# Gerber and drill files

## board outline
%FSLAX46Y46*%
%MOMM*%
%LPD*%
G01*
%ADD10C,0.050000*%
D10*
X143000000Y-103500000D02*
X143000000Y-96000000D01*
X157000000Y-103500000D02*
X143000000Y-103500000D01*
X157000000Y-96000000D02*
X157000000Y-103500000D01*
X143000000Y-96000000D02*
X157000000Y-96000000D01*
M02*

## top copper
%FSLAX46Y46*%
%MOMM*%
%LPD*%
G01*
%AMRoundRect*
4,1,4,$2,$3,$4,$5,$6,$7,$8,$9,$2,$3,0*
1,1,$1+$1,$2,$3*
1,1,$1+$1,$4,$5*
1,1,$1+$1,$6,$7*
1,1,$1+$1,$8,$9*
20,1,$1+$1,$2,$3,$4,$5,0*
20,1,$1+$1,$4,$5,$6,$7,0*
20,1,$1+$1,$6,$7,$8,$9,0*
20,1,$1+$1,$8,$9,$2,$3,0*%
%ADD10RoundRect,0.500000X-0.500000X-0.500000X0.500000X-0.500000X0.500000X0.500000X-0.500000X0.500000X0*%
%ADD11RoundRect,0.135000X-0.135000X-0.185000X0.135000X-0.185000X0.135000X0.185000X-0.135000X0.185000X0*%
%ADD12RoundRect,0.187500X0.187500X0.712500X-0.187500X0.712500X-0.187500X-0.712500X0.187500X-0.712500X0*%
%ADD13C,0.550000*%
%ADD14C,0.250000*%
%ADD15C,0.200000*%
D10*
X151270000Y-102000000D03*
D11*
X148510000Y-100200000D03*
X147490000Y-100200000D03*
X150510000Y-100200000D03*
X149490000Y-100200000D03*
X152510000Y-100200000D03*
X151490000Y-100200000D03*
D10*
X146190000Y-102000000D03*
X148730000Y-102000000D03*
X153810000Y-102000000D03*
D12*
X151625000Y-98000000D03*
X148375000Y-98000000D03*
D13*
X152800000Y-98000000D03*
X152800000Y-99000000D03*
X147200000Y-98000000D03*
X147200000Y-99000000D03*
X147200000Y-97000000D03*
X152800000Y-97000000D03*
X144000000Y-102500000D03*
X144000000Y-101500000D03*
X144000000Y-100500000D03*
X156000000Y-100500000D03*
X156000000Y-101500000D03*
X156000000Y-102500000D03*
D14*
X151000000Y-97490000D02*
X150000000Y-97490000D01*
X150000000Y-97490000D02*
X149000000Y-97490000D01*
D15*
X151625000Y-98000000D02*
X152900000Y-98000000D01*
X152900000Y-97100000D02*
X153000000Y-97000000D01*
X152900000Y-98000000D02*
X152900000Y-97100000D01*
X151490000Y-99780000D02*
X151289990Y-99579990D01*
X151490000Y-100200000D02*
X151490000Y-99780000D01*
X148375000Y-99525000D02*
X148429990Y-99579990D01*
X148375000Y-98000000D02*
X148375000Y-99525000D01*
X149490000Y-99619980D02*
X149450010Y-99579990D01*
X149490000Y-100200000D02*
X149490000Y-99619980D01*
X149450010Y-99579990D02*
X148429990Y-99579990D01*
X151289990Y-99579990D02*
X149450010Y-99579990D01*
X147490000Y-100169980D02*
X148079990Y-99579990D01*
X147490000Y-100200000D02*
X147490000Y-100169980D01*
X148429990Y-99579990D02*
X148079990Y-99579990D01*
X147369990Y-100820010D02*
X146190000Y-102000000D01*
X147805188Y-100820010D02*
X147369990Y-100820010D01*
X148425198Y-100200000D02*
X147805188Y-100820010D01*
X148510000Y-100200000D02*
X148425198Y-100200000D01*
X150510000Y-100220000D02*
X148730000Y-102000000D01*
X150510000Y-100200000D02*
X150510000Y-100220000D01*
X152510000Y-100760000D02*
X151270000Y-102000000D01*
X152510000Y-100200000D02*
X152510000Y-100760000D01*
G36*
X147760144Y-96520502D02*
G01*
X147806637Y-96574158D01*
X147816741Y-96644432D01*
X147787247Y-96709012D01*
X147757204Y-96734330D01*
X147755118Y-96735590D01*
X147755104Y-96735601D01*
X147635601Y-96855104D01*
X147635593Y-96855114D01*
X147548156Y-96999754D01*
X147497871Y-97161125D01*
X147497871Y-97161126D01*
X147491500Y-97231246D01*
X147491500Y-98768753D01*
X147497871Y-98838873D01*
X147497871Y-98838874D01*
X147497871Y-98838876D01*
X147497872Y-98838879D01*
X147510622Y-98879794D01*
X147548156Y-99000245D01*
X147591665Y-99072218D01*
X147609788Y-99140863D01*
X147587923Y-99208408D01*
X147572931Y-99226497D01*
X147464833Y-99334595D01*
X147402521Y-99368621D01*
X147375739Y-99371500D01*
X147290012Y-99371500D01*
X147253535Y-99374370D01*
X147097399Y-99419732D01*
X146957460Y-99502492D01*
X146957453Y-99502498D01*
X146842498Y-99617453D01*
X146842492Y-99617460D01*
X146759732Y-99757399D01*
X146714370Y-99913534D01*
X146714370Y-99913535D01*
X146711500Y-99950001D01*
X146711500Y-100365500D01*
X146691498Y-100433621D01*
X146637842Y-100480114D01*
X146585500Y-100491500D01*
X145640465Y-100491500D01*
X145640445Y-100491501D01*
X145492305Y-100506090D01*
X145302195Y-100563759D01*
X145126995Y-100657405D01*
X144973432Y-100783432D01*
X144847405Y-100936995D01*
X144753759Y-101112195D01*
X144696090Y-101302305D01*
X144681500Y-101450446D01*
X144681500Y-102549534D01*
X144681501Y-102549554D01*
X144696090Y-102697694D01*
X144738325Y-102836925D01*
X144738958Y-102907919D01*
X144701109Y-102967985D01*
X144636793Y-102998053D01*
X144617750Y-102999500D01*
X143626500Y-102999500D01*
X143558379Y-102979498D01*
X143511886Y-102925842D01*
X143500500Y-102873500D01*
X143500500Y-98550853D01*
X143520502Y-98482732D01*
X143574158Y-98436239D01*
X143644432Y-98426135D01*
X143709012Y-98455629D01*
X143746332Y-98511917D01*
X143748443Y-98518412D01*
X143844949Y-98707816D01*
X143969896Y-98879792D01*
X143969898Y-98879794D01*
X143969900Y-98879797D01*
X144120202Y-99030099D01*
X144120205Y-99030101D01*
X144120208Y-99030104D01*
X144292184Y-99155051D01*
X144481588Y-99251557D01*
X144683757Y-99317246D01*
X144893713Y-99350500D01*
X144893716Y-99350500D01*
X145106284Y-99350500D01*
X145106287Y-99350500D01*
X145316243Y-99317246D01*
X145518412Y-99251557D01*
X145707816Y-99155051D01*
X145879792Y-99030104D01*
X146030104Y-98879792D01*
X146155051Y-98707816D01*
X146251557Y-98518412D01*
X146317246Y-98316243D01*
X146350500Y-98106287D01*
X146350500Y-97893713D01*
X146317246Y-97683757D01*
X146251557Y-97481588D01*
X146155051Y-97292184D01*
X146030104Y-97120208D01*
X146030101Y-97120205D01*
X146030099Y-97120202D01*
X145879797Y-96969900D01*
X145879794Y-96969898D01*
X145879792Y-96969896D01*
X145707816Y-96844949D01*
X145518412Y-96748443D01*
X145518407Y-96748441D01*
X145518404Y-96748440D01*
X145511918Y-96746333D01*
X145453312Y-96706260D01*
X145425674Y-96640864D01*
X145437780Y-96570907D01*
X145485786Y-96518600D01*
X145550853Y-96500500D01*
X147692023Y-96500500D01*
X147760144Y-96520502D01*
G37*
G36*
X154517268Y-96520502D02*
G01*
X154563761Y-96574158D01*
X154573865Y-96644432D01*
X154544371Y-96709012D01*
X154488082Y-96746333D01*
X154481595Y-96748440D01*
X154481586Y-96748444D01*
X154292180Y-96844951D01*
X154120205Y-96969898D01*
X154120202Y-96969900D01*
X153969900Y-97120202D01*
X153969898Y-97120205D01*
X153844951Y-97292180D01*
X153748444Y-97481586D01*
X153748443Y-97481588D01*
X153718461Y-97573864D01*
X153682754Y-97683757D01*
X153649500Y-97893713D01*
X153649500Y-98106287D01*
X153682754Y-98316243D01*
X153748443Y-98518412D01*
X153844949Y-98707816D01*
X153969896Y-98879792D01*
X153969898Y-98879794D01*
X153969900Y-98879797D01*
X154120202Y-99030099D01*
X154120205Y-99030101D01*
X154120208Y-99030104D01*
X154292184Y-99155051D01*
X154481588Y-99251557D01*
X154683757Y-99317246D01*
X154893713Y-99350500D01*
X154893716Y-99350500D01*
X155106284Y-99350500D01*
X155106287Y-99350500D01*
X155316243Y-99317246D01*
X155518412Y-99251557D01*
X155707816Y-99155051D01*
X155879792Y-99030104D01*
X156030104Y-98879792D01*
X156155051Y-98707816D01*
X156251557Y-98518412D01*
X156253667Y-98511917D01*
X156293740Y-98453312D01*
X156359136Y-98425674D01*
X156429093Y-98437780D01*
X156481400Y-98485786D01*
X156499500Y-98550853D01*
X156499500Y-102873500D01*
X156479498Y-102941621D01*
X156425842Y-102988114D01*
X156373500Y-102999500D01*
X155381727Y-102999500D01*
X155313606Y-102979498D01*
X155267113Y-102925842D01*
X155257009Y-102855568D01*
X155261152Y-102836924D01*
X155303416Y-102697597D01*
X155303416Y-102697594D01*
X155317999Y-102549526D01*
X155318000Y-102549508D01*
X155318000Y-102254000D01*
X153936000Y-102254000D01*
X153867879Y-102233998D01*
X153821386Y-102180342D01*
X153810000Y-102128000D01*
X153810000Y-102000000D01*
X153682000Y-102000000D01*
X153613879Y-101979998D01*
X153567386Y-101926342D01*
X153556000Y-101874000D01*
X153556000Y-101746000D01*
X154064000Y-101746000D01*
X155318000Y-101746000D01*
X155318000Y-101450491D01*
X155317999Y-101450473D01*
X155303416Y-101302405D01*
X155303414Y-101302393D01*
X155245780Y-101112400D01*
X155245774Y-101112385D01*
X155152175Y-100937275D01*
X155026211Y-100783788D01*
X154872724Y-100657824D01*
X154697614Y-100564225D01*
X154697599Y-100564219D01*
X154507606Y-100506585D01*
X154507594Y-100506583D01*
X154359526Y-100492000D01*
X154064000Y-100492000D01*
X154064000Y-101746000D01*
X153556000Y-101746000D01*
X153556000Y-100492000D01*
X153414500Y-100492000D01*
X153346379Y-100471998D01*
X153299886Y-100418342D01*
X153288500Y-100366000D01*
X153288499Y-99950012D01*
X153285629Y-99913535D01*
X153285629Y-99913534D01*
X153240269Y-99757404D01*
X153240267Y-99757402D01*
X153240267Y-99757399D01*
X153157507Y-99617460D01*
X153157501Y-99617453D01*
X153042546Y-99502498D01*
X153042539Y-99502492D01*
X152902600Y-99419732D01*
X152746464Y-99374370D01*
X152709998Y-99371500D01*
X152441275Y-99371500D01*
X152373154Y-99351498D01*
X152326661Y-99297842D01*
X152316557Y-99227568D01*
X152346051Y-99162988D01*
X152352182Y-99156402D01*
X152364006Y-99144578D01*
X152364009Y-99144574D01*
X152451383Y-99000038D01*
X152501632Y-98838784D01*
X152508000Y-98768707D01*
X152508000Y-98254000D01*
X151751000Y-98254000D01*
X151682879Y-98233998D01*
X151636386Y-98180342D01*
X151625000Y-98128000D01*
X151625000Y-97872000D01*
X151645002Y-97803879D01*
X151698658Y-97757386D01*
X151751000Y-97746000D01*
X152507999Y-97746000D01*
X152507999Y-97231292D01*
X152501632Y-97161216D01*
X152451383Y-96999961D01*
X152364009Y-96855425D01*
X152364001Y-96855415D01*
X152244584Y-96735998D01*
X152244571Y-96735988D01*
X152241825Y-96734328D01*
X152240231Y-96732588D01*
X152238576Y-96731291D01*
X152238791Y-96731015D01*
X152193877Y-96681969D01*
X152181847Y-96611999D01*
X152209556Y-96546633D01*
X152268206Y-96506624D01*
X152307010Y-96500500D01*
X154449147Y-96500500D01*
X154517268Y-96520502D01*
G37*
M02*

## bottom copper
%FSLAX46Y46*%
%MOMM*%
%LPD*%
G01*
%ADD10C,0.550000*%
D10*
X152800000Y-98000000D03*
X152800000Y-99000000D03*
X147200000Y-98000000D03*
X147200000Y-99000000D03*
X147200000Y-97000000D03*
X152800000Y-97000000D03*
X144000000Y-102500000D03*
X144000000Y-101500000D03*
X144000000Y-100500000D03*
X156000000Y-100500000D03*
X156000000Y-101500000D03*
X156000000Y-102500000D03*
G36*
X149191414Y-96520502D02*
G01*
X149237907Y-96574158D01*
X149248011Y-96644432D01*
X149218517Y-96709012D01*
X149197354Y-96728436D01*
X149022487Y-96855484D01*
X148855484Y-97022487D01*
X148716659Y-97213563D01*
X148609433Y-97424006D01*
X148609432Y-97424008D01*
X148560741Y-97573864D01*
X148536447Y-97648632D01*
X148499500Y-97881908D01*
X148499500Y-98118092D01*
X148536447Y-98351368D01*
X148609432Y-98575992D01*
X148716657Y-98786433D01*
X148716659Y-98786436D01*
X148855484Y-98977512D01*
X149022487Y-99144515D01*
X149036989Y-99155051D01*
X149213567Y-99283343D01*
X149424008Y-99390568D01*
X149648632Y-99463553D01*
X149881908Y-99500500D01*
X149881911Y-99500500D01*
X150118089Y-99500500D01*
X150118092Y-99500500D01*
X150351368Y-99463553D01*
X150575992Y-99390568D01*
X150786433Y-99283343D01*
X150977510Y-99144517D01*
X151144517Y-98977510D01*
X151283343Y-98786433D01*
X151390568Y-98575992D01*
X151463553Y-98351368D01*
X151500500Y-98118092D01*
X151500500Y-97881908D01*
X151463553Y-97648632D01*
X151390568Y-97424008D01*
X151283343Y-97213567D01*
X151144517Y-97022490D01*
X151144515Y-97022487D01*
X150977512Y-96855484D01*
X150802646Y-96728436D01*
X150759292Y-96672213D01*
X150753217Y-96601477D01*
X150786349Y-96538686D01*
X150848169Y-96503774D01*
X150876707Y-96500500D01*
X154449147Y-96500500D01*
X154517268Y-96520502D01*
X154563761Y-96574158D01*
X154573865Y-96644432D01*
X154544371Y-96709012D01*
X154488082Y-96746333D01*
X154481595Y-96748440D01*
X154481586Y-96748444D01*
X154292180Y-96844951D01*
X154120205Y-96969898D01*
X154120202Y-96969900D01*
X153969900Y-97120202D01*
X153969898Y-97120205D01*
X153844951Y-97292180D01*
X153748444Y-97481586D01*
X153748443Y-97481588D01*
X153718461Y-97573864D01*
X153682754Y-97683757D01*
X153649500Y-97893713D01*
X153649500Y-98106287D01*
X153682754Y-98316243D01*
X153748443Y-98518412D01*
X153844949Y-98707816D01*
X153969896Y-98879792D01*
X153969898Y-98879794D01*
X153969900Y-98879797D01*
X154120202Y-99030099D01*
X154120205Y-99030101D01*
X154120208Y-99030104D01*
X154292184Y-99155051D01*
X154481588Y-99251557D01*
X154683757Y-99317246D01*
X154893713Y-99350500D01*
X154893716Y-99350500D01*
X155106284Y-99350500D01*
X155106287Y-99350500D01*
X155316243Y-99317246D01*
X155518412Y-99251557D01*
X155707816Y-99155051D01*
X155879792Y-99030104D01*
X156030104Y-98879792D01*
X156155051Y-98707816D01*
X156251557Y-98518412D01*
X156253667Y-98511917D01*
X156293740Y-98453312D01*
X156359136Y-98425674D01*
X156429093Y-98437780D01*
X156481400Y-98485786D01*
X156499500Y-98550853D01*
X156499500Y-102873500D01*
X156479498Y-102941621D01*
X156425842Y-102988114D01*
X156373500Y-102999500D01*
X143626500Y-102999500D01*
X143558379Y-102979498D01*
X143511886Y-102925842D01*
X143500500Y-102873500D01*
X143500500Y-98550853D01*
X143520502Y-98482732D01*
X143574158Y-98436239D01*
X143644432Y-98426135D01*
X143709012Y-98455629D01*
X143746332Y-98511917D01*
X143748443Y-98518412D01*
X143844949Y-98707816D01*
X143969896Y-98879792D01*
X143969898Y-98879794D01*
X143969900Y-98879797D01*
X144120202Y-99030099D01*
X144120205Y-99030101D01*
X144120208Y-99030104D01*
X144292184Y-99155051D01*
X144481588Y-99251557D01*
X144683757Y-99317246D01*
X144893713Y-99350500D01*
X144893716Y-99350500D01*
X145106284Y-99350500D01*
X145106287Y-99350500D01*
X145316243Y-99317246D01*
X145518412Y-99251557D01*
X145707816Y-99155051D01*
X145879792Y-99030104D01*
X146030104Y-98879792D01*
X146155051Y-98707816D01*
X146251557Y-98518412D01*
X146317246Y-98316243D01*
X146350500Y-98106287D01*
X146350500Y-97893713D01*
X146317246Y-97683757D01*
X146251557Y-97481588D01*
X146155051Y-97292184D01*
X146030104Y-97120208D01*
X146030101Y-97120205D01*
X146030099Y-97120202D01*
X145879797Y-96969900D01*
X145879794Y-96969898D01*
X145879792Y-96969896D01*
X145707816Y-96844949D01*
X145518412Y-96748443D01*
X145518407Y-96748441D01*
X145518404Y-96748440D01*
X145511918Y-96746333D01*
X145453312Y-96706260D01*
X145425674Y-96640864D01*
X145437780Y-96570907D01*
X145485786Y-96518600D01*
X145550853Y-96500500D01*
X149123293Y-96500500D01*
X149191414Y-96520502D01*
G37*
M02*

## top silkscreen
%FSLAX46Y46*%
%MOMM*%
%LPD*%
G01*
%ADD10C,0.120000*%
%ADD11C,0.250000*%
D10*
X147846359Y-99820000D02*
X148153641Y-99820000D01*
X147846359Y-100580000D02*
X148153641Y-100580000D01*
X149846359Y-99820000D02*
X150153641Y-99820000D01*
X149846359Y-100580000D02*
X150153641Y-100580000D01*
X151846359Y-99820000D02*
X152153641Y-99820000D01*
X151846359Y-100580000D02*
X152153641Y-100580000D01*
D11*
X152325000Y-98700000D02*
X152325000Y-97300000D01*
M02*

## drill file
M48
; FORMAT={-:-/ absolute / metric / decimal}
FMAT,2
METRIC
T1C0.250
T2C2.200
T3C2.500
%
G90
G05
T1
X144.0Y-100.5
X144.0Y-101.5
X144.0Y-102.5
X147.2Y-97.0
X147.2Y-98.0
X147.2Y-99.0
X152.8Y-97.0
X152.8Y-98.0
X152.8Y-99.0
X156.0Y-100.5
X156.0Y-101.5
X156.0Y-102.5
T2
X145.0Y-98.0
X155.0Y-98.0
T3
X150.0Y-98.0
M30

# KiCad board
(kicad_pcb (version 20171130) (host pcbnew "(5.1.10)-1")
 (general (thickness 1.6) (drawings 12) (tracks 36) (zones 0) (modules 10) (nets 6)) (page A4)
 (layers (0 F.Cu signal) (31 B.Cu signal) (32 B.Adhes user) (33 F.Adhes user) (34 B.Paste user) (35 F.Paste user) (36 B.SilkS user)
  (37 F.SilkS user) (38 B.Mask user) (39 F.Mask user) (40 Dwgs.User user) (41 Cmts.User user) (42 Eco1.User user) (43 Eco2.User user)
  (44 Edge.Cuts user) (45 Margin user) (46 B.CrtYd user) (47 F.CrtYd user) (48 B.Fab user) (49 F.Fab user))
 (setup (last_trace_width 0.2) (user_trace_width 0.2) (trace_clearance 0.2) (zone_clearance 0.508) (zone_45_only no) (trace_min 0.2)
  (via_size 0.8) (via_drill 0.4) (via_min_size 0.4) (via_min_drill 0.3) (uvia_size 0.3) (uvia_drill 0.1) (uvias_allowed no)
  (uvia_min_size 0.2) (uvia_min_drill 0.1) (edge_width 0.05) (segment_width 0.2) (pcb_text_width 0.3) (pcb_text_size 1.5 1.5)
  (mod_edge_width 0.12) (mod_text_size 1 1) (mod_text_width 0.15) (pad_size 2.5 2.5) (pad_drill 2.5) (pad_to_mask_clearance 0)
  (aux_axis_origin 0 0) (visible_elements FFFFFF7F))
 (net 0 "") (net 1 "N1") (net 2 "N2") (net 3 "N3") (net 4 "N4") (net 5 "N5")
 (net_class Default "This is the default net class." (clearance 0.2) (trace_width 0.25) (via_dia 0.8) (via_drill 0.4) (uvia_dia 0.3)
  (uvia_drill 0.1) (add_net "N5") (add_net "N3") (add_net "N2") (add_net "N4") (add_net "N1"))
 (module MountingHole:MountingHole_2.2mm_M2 (layer F.Cu) (at 145 98)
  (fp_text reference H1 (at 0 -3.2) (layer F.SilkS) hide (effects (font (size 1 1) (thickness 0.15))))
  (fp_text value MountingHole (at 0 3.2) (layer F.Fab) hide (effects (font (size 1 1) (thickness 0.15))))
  (pad 1 np_thru_hole circle (at 0 0) (size 2.2 2.2) (drill 2.2) (layers *.Cu *.Mask)))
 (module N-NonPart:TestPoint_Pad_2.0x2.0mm (layer F.Cu) (at 151.27 102)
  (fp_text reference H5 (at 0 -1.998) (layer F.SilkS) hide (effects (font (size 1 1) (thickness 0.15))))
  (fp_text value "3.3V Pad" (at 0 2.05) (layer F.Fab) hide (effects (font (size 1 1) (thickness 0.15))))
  (pad 1 smd roundrect (at 0 0) (size 2 2) (layers F.Cu F.Mask) (roundrect_rratio 0.25) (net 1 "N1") (solder_mask_margin 0.05)))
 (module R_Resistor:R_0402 (layer F.Cu) (at 148 100.2)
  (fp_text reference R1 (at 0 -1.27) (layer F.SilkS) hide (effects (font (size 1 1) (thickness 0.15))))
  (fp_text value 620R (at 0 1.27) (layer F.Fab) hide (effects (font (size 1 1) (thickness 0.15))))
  (fp_line (start -0.153641 -0.38) (end 0.153641 -0.38) (layer F.SilkS) (width 0.12))
  (fp_line (start -0.153641 0.38) (end 0.153641 0.38) (layer F.SilkS) (width 0.12))
  (pad 2 smd roundrect (at 0.51 0) (size 0.54 0.64) (layers F.Cu F.Paste F.Mask) (roundrect_rratio 0.25) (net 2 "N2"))
  (pad 1 smd roundrect (at -0.51 0) (size 0.54 0.64) (layers F.Cu F.Paste F.Mask) (roundrect_rratio 0.25) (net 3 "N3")))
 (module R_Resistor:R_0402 (layer F.Cu) (at 150 100.2)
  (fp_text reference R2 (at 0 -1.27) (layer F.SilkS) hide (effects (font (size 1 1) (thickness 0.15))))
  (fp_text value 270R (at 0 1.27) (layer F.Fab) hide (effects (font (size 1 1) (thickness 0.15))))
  (fp_line (start -0.153641 -0.38) (end 0.153641 -0.38) (layer F.SilkS) (width 0.12))
  (fp_line (start -0.153641 0.38) (end 0.153641 0.38) (layer F.SilkS) (width 0.12))
  (pad 2 smd roundrect (at 0.51 0) (size 0.54 0.64) (layers F.Cu F.Paste F.Mask) (roundrect_rratio 0.25) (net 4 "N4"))
  (pad 1 smd roundrect (at -0.51 0) (size 0.54 0.64) (layers F.Cu F.Paste F.Mask) (roundrect_rratio 0.25) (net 3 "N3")))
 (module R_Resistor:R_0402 (layer F.Cu) (at 152 100.2)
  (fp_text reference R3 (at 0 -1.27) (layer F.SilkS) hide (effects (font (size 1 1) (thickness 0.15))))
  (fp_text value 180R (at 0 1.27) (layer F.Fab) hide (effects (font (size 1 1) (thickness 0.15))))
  (fp_line (start -0.153641 -0.38) (end 0.153641 -0.38) (layer F.SilkS) (width 0.12))
  (fp_line (start -0.153641 0.38) (end 0.153641 0.38) (layer F.SilkS) (width 0.12))
  (pad 2 smd roundrect (at 0.51 0) (size 0.54 0.64) (layers F.Cu F.Paste F.Mask) (roundrect_rratio 0.25) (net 1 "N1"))
  (pad 1 smd roundrect (at -0.51 0) (size 0.54 0.64) (layers F.Cu F.Paste F.Mask) (roundrect_rratio 0.25) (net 3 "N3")))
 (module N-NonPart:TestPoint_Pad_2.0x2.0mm (layer F.Cu) (at 146.19 102)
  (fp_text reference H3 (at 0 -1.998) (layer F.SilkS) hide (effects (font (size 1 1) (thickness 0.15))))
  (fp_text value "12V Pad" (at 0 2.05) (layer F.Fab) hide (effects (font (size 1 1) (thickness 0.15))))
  (pad 1 smd roundrect (at 0 0) (size 2 2) (layers F.Cu F.Mask) (roundrect_rratio 0.25) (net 2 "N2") (solder_mask_margin 0.05)))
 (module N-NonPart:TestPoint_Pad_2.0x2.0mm (layer F.Cu) (at 148.73 102)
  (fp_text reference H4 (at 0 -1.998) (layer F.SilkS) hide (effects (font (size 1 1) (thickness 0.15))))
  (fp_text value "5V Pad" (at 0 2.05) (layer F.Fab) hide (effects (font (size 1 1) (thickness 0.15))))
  (pad 1 smd roundrect (at 0 0) (size 2 2) (layers F.Cu F.Mask) (roundrect_rratio 0.25) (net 4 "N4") (solder_mask_margin 0.05)))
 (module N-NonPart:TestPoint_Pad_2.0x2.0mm (layer F.Cu) (at 153.81 102)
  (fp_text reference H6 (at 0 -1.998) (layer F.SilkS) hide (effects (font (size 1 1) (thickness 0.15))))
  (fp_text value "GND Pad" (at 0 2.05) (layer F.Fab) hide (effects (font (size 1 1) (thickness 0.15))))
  (pad 1 smd roundrect (at 0 0) (size 2 2) (layers F.Cu F.Mask) (roundrect_rratio 0.25) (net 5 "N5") (solder_mask_margin 0.05)))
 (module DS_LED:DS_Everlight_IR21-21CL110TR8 (layer F.Cu) (at 150 98 180)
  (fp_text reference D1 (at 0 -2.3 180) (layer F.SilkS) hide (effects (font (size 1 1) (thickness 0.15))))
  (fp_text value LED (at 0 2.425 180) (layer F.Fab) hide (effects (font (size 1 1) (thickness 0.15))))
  (fp_line (start -2.325 -0.7) (end -2.325 0.7) (layer F.SilkS) (width 0.25))
  (pad "" np_thru_hole circle (at 0 0 180) (size 2.5 2.5) (drill 2.5) (layers *.Cu *.Mask) (solder_mask_margin 0.05))
  (pad 1 smd roundrect (at -1.625 0 180) (size 0.75 1.8) (layers F.Cu F.Paste F.Mask) (roundrect_rratio 0.25) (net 5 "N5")
   (solder_mask_margin 0.05) (solder_paste_margin -0.05))
  (pad 2 smd roundrect (at 1.625 0 180) (size 0.75 1.8) (layers F.Cu F.Paste F.Mask) (roundrect_rratio 0.25) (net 3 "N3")
   (solder_mask_margin 0.05) (solder_paste_margin -0.05)))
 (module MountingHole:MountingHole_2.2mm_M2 (layer F.Cu) (at 155 98)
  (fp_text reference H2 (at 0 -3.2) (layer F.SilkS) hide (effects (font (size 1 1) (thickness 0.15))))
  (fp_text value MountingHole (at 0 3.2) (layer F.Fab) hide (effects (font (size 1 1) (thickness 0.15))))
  (pad 1 np_thru_hole circle (at 0 0) (size 2.2 2.2) (drill 2.2) (layers *.Cu *.Mask)))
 (gr_line (start 143 103.5) (end 143 96) (layer Edge.Cuts) (width 0.05))
 (gr_line (start 157 103.5) (end 143 103.5) (layer Edge.Cuts) (width 0.05))
 (gr_line (start 157 96) (end 157 103.5) (layer Edge.Cuts) (width 0.05))
 (gr_line (start 143 96) (end 157 96) (layer Edge.Cuts) (width 0.05))
 (segment (start 151 97.49) (end 150 97.49) (width 0.25) (layer F.Cu) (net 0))
 (segment (start 150 97.49) (end 149 97.49) (width 0.25) (layer F.Cu) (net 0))
 (via (at 152.8 98) (size 0.55) (drill 0.25) (layers F.Cu B.Cu) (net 5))
 (via (at 152.8 99) (size 0.55) (drill 0.25) (layers F.Cu B.Cu) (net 5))
 (via (at 147.2 98) (size 0.55) (drill 0.25) (layers F.Cu B.Cu) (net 5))
 (via (at 147.2 99) (size 0.55) (drill 0.25) (layers F.Cu B.Cu) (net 5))
 (via (at 147.2 97) (size 0.55) (drill 0.25) (layers F.Cu B.Cu) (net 5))
 (via (at 152.8 97) (size 0.55) (drill 0.25) (layers F.Cu B.Cu) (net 5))
 (via (at 144 102.5) (size 0.55) (drill 0.25) (layers F.Cu B.Cu) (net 5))
 (via (at 144 101.5) (size 0.55) (drill 0.25) (layers F.Cu B.Cu) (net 5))
 (via (at 144 100.5) (size 0.55) (drill 0.25) (layers F.Cu B.Cu) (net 5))
 (via (at 156 100.5) (size 0.55) (drill 0.25) (layers F.Cu B.Cu) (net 5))
 (via (at 156 101.5) (size 0.55) (drill 0.25) (layers F.Cu B.Cu) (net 5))
 (via (at 156 102.5) (size 0.55) (drill 0.25) (layers F.Cu B.Cu) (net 5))
 (segment (start 151.625 98) (end 152.9 98) (width 0.2) (layer F.Cu) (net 5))
 (segment (start 152.9 97.1) (end 153 97) (width 0.2) (layer F.Cu) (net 5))
 (segment (start 152.9 98) (end 152.9 97.1) (width 0.2) (layer F.Cu) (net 5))
 (segment (start 151.49 99.78) (end 151.28999 99.57999) (width 0.2) (layer F.Cu) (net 3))
 (segment (start 151.49 100.2) (end 151.49 99.78) (width 0.2) (layer F.Cu) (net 3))
 (segment (start 148.375 99.525) (end 148.42999 99.57999) (width 0.2) (layer F.Cu) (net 3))
 (segment (start 148.375 98) (end 148.375 99.525) (width 0.2) (layer F.Cu) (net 3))
 (segment (start 149.49 99.61998) (end 149.45001 99.57999) (width 0.2) (layer F.Cu) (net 3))
 (segment (start 149.49 100.2) (end 149.49 99.61998) (width 0.2) (layer F.Cu) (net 3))
 (segment (start 149.45001 99.57999) (end 148.42999 99.57999) (width 0.2) (layer F.Cu) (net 3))
 (segment (start 151.28999 99.57999) (end 149.45001 99.57999) (width 0.2) (layer F.Cu) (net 3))
 (segment (start 147.49 100.16998) (end 148.07999 99.57999) (width 0.2) (layer F.Cu) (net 3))
 (segment (start 147.49 100.2) (end 147.49 100.16998) (width 0.2) (layer F.Cu) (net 3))
 (segment (start 148.42999 99.57999) (end 148.07999 99.57999) (width 0.2) (layer F.Cu) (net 3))
 (segment (start 147.36999 100.82001) (end 146.19 102) (width 0.2) (layer F.Cu) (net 2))
 (segment (start 147.805188 100.82001) (end 147.36999 100.82001) (width 0.2) (layer F.Cu) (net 2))
 (segment (start 148.425198 100.2) (end 147.805188 100.82001) (width 0.2) (layer F.Cu) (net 2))
 (segment (start 148.51 100.2) (end 148.425198 100.2) (width 0.2) (layer F.Cu) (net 2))
 (segment (start 150.51 100.22) (end 148.73 102) (width 0.2) (layer F.Cu) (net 4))
 (segment (start 150.51 100.2) (end 150.51 100.22) (width 0.2) (layer F.Cu) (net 4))
 (segment (start 152.51 100.76) (end 151.27 102) (width 0.2) (layer F.Cu) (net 1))
 (segment (start 152.51 100.2) (end 152.51 100.76) (width 0.2) (layer F.Cu) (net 1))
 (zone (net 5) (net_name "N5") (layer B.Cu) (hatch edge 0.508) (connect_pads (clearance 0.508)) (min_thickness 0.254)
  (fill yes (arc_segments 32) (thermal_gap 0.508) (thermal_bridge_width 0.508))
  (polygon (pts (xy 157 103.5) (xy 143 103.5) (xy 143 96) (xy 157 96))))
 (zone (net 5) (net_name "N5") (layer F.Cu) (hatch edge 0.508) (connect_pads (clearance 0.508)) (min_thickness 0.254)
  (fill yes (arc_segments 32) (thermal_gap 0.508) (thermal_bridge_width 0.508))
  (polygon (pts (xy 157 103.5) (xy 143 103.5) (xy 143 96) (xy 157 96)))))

